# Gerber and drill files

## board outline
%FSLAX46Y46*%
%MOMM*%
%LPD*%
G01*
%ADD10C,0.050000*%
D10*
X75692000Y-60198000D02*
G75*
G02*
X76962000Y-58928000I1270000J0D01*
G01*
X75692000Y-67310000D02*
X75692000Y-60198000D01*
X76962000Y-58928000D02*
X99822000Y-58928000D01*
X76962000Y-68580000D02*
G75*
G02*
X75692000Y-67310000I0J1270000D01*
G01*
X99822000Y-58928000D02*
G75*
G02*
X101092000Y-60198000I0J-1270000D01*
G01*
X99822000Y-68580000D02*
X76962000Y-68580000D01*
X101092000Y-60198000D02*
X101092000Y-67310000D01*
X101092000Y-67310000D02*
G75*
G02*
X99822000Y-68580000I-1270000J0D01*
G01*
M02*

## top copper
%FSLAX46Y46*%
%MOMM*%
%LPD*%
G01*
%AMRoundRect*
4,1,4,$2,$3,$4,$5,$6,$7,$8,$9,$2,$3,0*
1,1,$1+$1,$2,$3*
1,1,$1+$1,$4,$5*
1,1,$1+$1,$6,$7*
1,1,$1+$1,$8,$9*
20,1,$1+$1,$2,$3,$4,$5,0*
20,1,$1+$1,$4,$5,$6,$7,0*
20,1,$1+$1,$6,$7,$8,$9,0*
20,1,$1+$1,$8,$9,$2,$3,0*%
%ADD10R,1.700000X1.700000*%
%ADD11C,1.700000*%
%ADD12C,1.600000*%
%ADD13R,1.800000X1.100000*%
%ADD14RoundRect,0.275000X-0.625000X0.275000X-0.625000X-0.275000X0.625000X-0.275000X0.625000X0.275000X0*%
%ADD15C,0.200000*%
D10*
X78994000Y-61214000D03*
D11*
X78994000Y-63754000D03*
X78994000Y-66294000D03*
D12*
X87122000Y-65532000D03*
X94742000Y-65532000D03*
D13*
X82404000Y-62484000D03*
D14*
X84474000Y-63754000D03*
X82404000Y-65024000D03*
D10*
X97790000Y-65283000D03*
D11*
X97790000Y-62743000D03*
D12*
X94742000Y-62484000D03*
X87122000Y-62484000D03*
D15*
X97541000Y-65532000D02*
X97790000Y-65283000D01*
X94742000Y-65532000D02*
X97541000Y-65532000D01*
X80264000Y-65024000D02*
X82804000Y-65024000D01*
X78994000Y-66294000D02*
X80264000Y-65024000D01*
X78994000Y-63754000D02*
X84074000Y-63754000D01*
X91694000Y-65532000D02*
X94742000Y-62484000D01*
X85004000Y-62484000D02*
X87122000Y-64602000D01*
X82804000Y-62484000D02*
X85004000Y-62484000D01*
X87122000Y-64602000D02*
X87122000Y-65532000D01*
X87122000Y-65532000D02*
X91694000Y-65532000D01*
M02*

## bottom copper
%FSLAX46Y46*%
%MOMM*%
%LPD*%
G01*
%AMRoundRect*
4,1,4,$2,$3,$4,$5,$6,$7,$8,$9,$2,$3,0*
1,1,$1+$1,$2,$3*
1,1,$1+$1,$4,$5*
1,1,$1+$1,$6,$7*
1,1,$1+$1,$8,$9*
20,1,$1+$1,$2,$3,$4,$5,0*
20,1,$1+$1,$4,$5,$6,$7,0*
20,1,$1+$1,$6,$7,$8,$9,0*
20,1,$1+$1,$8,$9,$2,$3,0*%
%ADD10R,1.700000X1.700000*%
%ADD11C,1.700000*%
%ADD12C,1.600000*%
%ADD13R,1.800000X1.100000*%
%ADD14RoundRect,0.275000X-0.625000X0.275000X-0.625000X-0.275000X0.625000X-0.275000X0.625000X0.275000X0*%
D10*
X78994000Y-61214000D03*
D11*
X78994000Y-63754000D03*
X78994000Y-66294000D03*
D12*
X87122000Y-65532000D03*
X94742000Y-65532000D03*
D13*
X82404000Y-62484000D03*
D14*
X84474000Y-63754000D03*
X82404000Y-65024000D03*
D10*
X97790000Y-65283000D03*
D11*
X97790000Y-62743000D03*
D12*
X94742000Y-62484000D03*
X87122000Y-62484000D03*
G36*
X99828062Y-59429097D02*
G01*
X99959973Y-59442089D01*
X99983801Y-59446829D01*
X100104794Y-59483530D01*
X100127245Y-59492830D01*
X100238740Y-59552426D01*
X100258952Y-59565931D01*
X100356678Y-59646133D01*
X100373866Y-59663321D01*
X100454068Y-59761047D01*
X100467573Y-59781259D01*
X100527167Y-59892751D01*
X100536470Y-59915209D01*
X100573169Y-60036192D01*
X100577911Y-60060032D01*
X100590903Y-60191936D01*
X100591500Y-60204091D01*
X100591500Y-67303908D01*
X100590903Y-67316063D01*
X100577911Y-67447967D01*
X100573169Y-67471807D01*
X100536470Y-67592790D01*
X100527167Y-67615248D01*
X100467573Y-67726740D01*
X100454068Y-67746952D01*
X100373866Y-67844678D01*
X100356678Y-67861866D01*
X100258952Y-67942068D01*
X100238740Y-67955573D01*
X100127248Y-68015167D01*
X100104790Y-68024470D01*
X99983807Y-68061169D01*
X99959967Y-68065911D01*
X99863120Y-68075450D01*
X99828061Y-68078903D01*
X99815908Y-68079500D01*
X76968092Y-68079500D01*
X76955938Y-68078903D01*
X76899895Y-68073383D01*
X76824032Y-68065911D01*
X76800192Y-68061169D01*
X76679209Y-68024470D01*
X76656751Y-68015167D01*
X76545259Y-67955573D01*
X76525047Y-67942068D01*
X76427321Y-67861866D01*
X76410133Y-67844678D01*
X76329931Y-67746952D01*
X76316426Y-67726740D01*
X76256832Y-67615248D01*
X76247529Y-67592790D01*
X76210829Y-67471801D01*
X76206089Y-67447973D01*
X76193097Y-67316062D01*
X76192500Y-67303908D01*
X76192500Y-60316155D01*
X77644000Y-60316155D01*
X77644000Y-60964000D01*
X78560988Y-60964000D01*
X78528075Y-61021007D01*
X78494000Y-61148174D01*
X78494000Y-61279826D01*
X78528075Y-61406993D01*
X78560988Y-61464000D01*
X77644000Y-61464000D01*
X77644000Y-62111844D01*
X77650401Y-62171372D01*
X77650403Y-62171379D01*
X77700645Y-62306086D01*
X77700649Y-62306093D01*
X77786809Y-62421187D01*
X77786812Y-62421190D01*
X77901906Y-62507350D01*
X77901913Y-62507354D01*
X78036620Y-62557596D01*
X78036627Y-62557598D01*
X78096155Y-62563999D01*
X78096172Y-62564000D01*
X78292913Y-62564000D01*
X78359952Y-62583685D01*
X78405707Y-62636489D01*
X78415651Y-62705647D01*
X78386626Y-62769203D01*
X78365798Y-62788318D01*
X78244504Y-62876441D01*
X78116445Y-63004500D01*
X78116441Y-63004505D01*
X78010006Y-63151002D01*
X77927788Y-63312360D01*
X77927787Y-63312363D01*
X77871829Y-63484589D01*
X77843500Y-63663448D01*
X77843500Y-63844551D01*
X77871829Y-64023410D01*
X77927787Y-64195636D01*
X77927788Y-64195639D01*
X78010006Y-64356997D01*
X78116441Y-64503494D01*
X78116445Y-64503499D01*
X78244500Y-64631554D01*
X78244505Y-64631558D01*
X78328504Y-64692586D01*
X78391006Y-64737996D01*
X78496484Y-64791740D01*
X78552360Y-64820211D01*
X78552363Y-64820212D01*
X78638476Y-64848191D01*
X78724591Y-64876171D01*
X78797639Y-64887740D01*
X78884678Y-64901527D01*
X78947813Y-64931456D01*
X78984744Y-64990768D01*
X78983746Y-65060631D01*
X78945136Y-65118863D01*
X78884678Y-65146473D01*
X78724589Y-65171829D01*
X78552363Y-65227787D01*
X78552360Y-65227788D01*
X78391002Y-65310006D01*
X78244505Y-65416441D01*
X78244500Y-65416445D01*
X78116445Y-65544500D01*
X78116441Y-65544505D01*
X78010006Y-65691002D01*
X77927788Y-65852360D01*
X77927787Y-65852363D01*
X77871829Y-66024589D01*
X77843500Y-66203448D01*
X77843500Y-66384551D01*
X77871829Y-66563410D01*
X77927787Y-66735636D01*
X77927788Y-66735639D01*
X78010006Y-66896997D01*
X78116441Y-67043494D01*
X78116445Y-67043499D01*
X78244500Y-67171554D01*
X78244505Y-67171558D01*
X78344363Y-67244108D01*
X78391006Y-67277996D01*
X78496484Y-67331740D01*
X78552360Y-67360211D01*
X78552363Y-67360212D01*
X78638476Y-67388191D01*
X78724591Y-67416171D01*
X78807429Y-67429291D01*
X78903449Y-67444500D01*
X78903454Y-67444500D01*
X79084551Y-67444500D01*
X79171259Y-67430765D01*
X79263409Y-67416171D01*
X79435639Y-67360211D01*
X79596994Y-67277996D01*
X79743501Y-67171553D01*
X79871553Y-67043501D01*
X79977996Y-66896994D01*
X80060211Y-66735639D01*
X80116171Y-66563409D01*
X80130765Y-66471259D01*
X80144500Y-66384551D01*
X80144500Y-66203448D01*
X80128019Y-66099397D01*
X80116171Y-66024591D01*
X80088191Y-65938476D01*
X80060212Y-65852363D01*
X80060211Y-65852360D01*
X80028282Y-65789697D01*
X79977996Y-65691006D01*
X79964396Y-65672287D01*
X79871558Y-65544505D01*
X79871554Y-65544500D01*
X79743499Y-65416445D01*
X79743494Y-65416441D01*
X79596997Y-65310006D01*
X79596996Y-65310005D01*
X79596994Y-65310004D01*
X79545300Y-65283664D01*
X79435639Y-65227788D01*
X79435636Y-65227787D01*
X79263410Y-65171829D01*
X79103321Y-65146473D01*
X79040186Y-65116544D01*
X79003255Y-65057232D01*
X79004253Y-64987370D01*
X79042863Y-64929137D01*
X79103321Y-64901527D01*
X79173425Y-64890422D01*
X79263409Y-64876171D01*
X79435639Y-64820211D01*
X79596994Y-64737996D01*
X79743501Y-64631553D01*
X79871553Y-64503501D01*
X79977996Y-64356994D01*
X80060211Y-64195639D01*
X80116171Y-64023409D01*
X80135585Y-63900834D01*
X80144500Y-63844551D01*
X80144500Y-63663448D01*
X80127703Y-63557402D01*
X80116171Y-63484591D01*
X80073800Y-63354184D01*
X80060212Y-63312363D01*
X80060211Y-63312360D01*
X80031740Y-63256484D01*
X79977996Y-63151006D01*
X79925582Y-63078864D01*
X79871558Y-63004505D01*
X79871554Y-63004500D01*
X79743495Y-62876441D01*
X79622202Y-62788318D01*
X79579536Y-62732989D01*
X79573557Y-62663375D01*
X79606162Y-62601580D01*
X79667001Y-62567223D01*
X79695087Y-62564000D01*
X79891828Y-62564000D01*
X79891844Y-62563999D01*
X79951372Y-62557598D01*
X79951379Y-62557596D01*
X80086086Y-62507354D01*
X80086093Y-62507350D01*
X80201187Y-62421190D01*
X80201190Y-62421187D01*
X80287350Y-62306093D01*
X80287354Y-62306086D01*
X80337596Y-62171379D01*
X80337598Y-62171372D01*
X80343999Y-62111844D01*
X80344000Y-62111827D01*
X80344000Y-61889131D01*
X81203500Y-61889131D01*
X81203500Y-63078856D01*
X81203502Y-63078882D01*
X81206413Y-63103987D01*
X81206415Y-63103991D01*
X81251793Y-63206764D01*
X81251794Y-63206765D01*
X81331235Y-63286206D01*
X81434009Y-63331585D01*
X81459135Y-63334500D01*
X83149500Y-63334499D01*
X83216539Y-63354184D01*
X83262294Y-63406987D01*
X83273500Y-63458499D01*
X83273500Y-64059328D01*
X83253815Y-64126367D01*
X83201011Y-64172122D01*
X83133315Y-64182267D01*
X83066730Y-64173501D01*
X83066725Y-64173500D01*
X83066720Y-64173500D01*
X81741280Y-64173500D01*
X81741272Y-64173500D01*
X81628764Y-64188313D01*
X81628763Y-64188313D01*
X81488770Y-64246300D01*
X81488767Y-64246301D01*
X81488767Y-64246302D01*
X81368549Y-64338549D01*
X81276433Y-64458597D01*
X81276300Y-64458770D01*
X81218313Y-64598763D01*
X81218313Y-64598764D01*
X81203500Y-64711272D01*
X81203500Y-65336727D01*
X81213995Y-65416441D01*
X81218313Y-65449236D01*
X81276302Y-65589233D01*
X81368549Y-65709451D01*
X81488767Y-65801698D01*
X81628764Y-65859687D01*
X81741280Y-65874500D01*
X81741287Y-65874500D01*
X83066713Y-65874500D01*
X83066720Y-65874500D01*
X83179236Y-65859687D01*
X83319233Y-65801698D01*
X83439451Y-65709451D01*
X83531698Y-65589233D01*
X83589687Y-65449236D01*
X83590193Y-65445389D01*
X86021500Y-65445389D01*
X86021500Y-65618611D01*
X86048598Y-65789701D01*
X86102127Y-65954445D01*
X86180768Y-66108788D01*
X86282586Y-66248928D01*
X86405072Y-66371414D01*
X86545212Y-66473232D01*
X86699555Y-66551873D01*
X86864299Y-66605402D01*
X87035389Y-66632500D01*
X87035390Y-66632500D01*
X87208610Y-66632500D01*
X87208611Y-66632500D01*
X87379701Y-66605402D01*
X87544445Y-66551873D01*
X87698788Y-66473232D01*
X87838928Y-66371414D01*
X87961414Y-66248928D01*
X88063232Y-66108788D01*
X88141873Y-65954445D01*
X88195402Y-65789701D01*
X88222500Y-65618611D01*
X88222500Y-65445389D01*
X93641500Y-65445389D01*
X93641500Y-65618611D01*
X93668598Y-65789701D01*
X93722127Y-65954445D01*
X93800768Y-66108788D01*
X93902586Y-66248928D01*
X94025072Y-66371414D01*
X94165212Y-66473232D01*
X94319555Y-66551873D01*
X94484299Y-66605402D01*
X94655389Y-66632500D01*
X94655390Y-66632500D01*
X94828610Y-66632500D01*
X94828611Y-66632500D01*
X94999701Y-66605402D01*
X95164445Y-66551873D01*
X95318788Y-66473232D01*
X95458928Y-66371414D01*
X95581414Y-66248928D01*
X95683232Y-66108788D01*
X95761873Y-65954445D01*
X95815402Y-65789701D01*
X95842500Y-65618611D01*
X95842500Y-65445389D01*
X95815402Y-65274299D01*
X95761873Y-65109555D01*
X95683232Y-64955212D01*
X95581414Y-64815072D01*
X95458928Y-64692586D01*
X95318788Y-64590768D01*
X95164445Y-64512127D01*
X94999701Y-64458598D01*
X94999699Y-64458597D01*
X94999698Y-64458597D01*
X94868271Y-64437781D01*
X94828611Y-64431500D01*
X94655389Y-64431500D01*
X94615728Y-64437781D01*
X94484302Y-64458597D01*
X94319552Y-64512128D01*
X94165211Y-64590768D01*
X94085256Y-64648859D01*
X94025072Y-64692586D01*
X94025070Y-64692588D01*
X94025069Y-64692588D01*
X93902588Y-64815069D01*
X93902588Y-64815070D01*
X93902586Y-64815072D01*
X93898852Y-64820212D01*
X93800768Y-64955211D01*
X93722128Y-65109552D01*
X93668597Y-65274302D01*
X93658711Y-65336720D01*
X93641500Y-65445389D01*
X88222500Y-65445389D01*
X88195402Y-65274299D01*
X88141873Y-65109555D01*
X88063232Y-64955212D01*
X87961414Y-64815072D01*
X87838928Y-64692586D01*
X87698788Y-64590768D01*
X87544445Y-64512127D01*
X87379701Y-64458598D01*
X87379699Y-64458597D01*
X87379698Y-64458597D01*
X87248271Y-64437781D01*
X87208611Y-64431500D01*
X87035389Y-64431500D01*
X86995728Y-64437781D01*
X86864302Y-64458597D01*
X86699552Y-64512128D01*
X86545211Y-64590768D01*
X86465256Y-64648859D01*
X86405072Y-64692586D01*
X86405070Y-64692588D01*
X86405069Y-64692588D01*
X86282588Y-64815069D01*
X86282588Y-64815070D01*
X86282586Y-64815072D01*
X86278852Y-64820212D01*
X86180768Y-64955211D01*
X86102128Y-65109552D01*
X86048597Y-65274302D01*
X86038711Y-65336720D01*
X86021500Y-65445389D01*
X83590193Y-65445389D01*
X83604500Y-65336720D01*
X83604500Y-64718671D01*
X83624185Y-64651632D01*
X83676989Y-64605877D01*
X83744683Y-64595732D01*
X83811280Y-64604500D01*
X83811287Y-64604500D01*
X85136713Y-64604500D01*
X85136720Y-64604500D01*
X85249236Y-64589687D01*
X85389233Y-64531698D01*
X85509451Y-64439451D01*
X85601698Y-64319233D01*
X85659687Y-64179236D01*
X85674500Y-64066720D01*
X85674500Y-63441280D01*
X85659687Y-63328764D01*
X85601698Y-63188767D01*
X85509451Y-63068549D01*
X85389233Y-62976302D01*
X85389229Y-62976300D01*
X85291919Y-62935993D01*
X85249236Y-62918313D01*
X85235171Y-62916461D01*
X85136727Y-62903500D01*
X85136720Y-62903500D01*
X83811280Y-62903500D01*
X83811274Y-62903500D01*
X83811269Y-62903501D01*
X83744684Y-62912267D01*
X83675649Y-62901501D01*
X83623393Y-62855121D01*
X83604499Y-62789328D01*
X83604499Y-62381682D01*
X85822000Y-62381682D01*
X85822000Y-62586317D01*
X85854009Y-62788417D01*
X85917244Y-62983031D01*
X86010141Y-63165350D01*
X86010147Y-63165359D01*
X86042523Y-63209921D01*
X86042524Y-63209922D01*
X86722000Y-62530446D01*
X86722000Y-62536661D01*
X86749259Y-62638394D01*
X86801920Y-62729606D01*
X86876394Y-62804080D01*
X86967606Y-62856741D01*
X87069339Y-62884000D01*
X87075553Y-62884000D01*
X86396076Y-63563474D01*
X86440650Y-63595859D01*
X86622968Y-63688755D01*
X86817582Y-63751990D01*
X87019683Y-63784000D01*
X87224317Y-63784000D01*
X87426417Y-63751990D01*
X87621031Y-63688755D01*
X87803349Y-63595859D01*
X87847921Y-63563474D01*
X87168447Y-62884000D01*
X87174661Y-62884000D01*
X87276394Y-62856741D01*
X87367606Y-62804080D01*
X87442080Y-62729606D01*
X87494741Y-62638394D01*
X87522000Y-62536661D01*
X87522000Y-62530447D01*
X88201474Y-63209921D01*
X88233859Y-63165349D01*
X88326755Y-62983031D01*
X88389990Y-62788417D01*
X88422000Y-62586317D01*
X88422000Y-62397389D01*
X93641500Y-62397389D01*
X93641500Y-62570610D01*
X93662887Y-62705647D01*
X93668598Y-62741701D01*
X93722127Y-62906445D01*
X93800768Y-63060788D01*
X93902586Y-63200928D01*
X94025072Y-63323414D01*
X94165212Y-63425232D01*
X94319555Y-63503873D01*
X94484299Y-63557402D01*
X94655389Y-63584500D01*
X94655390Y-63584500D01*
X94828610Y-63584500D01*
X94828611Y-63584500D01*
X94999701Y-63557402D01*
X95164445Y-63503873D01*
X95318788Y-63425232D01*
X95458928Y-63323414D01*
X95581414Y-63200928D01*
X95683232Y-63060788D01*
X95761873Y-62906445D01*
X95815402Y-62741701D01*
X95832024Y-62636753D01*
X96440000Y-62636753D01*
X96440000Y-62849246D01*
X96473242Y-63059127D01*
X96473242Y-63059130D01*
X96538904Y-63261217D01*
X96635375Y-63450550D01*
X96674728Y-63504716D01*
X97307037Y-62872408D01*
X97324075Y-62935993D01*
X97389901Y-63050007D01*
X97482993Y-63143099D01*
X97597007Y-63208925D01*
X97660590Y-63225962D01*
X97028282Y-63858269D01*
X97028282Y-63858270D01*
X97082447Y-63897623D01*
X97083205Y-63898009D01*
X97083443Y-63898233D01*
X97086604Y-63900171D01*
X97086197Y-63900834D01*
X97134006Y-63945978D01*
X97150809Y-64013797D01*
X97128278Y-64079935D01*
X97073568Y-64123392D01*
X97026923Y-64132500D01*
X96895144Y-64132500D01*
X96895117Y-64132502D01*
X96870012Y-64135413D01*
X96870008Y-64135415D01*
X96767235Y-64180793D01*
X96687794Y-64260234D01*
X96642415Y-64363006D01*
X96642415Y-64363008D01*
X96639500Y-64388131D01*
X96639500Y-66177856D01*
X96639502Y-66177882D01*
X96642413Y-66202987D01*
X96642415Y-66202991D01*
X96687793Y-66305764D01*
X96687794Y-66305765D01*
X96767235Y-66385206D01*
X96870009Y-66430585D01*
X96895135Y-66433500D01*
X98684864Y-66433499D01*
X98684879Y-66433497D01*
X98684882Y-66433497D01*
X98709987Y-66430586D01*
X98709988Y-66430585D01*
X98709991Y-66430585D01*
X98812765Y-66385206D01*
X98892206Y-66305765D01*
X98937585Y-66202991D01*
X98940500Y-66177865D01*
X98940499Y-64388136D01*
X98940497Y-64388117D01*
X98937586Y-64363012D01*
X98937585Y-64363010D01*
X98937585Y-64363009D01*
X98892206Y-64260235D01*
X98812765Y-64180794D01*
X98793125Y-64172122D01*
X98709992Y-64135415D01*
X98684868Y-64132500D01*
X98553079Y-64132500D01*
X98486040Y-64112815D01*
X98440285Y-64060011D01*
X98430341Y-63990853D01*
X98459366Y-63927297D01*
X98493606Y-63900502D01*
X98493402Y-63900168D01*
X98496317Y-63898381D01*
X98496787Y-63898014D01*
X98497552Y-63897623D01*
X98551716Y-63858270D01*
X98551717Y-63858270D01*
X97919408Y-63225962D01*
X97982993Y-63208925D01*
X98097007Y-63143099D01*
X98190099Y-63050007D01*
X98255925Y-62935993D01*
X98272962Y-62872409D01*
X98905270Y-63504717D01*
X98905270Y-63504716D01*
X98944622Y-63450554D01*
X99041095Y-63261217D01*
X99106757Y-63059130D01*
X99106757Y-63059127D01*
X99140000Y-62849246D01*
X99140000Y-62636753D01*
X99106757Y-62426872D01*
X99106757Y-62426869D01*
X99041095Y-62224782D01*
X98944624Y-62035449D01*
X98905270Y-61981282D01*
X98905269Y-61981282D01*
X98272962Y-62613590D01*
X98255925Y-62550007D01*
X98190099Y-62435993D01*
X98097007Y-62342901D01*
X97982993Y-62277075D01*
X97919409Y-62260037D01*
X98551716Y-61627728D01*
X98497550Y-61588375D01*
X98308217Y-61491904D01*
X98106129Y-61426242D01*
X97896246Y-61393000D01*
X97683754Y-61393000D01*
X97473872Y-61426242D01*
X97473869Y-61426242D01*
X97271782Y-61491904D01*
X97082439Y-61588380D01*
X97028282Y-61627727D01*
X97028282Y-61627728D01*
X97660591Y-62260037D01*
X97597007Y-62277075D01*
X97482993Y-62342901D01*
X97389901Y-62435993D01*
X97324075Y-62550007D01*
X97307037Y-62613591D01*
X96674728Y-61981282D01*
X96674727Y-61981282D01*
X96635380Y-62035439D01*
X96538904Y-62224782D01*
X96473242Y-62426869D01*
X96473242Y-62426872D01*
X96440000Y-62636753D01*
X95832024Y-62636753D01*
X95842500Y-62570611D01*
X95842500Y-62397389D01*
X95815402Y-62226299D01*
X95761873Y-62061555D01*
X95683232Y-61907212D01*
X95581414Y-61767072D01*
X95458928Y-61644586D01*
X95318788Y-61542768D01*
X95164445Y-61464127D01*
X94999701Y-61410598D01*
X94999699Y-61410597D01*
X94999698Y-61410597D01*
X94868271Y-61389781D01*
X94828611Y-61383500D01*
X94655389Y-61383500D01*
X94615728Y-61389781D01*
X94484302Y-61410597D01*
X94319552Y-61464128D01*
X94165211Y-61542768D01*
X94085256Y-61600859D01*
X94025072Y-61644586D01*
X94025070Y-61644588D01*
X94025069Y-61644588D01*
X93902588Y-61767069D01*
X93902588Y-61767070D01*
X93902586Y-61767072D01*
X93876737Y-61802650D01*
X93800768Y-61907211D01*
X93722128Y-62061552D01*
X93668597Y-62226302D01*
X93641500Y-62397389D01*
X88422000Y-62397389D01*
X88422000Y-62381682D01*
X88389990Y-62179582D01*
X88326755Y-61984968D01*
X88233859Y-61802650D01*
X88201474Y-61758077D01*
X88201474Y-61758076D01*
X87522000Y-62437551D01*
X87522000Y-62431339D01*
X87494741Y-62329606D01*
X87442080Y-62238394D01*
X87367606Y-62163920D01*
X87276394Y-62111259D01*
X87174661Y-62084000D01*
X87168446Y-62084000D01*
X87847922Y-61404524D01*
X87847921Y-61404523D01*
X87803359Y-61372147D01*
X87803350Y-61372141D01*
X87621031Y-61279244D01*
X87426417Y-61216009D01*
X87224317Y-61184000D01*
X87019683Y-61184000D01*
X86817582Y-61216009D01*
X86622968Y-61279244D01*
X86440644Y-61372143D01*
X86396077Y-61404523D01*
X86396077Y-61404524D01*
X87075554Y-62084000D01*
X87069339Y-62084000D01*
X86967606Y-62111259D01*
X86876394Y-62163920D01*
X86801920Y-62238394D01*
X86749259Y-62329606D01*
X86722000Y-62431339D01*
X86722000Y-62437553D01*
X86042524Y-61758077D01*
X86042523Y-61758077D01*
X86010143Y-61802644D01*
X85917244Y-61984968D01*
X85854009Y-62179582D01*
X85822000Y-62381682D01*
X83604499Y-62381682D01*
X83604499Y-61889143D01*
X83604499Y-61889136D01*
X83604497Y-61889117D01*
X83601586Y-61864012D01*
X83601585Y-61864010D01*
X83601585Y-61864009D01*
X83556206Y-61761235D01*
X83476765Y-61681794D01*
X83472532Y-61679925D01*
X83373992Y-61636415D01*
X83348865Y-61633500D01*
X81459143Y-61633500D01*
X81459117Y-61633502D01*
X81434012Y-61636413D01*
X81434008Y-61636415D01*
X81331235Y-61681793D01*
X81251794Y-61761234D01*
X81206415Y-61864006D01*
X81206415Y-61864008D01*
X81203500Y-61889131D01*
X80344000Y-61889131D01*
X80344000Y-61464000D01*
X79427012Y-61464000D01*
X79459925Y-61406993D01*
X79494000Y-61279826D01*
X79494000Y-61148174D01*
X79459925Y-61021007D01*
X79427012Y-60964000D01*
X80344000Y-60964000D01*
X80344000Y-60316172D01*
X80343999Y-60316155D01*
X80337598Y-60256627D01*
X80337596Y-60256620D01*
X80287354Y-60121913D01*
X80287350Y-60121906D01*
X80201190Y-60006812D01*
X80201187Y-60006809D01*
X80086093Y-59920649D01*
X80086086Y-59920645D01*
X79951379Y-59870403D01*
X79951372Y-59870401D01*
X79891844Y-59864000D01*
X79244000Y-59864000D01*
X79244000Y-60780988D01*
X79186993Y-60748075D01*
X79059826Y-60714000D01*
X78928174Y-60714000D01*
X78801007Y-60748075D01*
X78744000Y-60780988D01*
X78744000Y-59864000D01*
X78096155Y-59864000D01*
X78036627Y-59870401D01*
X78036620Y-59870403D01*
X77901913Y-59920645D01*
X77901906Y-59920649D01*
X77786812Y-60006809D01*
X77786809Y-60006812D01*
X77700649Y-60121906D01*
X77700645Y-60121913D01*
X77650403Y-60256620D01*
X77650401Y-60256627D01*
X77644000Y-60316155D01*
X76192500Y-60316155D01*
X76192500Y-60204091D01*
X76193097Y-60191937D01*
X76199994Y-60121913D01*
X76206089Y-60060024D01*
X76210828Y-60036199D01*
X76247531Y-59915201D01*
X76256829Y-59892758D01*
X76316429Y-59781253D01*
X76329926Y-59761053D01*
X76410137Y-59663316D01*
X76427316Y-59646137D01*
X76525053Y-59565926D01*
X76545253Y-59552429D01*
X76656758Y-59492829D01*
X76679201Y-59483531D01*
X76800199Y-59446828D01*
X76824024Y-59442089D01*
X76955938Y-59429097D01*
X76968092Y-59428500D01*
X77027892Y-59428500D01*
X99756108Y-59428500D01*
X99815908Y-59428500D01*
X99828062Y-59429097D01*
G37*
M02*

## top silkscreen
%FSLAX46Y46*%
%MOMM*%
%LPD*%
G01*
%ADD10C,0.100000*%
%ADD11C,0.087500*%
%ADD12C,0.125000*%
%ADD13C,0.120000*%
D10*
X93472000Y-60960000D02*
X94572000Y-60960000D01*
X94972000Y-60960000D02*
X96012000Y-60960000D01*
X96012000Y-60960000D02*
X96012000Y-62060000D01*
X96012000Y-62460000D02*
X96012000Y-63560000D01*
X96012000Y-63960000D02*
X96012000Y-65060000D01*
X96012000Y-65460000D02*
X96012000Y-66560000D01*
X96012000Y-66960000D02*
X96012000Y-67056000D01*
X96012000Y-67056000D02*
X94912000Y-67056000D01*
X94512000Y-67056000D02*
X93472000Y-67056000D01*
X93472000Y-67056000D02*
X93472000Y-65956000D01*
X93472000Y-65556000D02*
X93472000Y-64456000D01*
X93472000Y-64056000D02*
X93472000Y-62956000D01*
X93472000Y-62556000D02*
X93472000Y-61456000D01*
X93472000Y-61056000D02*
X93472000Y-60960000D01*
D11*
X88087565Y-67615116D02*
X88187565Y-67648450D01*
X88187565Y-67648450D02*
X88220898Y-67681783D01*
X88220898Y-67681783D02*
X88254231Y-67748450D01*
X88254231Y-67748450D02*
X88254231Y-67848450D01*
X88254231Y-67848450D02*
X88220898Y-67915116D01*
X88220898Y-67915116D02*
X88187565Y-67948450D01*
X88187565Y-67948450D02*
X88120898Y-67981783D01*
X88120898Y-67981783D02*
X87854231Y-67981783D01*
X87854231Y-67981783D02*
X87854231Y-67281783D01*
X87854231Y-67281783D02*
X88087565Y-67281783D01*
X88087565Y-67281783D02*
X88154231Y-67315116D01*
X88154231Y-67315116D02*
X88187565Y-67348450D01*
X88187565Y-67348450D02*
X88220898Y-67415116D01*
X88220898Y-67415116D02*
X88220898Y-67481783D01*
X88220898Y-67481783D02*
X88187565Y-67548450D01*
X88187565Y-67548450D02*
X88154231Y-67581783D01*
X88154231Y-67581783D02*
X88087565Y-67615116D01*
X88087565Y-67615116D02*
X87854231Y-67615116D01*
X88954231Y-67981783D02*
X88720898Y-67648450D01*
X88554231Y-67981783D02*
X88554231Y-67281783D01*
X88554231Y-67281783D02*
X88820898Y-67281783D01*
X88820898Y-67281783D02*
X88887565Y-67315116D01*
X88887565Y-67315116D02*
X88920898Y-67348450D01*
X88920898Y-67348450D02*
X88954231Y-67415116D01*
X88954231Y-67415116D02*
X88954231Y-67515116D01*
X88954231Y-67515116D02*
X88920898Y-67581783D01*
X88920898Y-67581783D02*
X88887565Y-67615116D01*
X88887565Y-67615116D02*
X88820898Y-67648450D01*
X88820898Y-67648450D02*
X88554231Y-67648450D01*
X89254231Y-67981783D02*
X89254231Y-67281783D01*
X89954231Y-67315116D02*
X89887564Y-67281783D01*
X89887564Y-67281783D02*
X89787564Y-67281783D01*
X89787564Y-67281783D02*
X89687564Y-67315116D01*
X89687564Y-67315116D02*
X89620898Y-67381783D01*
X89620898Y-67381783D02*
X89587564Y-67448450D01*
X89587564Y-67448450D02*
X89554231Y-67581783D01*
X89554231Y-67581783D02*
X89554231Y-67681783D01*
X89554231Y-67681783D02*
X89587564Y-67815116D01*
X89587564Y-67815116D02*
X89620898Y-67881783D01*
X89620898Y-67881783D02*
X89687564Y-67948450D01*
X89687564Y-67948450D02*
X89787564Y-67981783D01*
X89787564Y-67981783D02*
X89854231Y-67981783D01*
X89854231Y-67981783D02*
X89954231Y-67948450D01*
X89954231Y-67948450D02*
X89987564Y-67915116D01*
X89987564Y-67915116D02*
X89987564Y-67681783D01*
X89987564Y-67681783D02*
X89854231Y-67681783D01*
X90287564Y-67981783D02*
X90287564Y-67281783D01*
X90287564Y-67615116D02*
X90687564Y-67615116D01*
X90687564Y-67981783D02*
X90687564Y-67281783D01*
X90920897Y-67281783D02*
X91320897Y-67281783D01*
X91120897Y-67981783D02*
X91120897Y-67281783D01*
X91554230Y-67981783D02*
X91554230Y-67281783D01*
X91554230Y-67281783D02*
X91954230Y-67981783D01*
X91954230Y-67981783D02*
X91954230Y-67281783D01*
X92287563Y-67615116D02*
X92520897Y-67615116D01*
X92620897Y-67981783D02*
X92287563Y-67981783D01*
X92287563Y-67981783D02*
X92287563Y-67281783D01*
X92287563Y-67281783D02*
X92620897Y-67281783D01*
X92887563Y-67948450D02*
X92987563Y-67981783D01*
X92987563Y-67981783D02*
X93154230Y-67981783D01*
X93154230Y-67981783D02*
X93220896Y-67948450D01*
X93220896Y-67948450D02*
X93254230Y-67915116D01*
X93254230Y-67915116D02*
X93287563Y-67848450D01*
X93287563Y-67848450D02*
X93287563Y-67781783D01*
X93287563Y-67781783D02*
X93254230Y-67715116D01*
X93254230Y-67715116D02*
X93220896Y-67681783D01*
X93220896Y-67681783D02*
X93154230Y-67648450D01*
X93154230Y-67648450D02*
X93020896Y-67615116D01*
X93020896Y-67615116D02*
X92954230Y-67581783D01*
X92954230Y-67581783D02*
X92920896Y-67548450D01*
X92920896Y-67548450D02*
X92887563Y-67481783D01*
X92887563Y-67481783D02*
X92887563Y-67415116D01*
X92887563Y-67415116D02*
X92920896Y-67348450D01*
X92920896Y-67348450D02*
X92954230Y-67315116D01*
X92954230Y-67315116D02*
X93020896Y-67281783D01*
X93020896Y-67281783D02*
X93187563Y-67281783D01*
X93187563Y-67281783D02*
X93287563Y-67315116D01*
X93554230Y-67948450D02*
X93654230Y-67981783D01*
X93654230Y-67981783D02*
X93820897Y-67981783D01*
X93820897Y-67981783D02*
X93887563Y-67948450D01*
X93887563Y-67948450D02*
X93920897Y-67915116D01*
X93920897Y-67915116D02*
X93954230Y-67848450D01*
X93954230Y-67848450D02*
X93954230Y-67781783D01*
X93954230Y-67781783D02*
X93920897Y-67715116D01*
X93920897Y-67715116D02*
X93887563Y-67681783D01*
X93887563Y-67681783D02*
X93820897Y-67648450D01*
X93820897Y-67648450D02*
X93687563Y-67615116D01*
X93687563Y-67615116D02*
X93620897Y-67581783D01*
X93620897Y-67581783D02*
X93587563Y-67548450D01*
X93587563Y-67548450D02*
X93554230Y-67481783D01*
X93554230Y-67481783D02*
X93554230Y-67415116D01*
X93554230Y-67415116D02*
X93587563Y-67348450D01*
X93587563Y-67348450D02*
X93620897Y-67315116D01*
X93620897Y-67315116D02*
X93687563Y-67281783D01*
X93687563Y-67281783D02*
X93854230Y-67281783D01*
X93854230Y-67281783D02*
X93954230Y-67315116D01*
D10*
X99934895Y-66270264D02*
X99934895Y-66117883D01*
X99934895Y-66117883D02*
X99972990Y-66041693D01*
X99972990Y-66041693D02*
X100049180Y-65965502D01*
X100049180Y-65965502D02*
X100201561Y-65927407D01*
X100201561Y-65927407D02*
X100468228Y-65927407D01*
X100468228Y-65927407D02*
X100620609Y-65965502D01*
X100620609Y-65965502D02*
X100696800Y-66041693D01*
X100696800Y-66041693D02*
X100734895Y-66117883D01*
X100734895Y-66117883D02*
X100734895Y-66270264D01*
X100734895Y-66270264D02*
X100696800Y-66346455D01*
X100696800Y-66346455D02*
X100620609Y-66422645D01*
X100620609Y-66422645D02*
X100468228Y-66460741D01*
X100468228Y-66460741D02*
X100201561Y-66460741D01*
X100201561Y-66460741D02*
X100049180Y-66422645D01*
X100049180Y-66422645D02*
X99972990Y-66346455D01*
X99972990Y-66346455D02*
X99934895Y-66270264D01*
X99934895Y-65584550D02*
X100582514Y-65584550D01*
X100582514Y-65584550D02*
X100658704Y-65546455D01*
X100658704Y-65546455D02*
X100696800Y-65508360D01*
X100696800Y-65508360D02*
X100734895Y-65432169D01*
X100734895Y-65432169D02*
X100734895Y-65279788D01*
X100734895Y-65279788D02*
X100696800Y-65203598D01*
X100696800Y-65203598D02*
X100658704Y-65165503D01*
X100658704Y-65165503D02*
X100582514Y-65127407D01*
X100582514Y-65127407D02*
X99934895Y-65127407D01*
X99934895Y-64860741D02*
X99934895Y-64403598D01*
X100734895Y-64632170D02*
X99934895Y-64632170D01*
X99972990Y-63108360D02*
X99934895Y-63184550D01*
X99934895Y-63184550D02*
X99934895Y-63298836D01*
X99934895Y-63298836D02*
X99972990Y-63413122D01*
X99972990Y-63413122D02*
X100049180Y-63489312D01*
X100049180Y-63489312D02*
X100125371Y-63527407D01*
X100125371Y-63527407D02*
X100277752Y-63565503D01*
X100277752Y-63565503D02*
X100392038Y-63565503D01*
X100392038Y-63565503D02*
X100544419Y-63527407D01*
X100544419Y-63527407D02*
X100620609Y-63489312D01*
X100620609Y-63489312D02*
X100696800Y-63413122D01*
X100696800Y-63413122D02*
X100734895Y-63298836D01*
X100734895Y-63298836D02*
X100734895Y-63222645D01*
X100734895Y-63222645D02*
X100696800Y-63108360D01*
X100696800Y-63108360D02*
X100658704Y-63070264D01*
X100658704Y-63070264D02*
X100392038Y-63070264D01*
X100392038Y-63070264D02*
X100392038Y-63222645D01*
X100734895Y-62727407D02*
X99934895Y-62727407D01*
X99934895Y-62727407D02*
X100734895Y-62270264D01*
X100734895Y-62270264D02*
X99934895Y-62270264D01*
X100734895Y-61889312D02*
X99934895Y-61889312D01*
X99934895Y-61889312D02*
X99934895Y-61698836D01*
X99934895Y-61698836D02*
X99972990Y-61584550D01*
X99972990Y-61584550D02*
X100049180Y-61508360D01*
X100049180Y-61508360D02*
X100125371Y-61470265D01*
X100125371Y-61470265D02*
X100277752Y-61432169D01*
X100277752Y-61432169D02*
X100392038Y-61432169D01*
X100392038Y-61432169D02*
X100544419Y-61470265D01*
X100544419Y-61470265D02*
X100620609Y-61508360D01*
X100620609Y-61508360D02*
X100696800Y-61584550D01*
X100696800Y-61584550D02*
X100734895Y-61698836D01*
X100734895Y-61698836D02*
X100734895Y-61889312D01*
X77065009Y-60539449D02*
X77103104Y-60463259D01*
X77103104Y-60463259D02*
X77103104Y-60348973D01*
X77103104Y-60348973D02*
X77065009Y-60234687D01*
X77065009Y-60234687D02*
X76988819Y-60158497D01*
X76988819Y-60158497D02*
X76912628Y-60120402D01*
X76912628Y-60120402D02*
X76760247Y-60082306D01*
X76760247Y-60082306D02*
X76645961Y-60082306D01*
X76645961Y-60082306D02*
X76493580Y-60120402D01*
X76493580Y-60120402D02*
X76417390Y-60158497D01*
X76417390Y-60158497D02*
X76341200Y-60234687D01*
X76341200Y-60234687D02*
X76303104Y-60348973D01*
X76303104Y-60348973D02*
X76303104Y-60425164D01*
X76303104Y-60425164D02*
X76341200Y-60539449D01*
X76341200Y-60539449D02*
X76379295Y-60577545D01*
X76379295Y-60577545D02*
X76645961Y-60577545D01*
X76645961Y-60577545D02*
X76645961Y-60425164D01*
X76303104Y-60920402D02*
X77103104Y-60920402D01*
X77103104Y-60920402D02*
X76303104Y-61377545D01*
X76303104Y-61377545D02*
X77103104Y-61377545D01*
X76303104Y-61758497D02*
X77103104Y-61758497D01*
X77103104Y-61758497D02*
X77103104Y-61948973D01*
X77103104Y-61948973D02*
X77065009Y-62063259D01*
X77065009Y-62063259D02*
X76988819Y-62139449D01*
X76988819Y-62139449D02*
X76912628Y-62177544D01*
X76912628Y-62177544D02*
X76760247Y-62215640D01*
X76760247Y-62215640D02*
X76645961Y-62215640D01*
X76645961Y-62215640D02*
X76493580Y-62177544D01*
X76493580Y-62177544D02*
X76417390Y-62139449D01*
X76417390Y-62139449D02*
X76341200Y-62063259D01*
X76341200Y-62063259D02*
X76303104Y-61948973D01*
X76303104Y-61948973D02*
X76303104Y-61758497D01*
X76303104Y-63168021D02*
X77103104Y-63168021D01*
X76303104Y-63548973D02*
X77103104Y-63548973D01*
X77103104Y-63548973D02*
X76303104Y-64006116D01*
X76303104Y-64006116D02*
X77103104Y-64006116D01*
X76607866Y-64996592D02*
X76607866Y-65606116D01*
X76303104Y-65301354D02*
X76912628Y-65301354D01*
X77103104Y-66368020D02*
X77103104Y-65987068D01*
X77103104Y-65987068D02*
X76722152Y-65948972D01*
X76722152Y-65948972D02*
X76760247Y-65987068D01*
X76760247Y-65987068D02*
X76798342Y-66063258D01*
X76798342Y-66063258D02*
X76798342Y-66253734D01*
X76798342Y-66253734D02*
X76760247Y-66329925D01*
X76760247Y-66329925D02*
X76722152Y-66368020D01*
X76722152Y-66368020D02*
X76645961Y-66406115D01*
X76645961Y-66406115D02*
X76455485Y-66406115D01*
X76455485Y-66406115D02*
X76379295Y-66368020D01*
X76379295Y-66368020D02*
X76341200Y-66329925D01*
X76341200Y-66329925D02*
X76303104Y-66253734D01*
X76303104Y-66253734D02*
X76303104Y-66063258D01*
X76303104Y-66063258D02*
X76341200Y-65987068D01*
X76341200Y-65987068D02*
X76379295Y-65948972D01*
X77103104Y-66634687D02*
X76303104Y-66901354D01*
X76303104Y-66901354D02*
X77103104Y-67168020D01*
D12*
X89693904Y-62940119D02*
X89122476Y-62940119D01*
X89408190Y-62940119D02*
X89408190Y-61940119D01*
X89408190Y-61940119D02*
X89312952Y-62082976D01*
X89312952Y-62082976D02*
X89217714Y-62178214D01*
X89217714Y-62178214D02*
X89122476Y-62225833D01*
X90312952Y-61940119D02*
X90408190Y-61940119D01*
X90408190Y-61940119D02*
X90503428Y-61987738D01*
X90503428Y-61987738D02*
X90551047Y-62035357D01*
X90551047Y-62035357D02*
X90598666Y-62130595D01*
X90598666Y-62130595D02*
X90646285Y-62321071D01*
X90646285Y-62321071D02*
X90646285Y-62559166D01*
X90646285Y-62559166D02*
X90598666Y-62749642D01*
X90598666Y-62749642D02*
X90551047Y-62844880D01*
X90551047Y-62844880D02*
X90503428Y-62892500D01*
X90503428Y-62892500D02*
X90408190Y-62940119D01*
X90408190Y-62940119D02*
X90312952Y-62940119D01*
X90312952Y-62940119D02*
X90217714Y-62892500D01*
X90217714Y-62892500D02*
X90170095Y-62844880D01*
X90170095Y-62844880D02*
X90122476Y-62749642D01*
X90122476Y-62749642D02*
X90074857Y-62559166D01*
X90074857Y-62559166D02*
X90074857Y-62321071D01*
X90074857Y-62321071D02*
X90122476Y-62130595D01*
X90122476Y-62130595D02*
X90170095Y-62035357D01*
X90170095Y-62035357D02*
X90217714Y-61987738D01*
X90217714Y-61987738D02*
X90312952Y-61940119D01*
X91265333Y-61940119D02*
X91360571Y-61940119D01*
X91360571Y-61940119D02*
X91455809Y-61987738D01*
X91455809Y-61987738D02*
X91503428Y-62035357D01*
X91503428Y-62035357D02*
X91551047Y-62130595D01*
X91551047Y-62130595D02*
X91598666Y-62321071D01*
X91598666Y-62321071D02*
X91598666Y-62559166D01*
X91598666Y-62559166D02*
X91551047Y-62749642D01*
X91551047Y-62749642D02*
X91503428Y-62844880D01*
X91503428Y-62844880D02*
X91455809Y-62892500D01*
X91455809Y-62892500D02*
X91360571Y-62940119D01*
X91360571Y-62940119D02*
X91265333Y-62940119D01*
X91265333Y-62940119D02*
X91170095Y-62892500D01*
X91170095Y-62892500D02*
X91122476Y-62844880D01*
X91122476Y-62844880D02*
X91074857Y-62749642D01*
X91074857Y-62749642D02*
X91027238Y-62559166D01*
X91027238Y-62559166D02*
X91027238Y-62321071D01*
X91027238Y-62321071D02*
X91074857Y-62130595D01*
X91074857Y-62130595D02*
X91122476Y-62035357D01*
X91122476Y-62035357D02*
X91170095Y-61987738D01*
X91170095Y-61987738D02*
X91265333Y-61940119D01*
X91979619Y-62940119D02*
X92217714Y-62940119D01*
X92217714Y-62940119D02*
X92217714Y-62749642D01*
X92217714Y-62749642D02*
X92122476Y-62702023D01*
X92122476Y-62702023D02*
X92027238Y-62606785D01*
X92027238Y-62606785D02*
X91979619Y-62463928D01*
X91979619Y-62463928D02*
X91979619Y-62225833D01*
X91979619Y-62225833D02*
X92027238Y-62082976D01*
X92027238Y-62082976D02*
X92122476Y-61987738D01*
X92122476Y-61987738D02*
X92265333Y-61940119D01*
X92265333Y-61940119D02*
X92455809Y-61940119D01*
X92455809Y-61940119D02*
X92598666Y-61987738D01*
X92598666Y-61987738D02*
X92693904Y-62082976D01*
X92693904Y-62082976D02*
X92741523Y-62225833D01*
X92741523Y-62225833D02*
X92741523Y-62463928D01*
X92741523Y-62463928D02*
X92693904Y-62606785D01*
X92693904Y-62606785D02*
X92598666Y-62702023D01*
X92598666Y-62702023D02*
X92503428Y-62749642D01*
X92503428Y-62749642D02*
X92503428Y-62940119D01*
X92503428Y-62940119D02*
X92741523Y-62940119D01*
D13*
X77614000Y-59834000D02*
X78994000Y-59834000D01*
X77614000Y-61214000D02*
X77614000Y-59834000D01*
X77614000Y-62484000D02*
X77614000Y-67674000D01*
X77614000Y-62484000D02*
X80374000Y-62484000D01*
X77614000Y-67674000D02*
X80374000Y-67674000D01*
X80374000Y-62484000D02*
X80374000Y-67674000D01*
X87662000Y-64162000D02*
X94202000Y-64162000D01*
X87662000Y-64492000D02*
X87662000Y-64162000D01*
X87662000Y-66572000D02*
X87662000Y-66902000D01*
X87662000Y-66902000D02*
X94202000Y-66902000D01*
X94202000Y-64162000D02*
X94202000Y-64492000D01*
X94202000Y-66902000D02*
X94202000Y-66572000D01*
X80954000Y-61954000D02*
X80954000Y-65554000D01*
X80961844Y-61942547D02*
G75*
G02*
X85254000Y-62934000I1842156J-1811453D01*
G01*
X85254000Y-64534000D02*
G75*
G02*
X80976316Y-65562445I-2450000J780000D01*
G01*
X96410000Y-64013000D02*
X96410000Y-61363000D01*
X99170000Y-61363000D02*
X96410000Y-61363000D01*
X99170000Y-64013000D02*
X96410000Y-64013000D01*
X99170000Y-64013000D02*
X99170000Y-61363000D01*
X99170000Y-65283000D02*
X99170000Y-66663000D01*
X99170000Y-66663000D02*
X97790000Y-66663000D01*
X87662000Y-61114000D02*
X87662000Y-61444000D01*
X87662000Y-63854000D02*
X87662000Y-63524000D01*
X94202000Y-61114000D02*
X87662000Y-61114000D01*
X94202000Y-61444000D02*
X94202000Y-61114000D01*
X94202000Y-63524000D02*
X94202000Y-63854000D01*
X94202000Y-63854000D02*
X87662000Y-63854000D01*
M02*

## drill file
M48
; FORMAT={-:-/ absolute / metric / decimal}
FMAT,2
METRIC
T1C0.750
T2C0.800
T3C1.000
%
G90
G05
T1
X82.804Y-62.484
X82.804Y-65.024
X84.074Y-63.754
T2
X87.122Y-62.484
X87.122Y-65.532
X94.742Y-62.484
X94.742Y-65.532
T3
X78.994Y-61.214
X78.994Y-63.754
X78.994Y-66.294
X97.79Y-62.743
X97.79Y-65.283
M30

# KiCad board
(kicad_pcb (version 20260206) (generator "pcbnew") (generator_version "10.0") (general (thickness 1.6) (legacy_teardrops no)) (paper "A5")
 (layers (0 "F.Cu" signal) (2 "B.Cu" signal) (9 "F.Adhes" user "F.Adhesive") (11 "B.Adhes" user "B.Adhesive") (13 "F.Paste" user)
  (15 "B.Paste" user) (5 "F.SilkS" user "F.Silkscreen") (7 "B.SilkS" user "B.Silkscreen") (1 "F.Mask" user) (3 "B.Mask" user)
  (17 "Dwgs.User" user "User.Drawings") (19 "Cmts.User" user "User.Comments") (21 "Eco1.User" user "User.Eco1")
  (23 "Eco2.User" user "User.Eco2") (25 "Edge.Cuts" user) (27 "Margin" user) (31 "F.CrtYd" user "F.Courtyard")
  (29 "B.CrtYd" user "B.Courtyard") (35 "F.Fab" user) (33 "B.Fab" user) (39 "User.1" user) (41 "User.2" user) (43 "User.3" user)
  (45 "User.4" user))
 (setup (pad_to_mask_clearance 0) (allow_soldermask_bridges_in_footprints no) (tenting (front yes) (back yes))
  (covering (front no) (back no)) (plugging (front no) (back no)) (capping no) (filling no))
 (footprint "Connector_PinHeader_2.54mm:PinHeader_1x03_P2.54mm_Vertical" (layer "F.Cu") (at 78.994 61.214)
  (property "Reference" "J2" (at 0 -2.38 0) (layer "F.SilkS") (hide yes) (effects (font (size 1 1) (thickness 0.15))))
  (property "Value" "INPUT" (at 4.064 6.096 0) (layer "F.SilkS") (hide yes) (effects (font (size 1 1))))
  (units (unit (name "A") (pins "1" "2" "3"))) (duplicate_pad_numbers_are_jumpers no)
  (fp_line (start -1.38 -1.38) (end 0 -1.38) (stroke (width 0.12) (type solid)) (layer "F.SilkS"))
  (fp_line (start -1.38 0) (end -1.38 -1.38) (stroke (width 0.12) (type solid)) (layer "F.SilkS"))
  (fp_line (start -1.38 1.27) (end -1.38 6.46) (stroke (width 0.12) (type solid)) (layer "F.SilkS"))
  (fp_line (start -1.38 1.27) (end 1.38 1.27) (stroke (width 0.12) (type solid)) (layer "F.SilkS"))
  (fp_line (start -1.38 6.46) (end 1.38 6.46) (stroke (width 0.12) (type solid)) (layer "F.SilkS"))
  (fp_line (start 1.38 1.27) (end 1.38 6.46) (stroke (width 0.12) (type solid)) (layer "F.SilkS"))
  (pad "1" thru_hole rect (at 0 0) (size 1.7 1.7) (drill 1) (layers "*.Cu" "*.Mask") (remove_unused_layers no) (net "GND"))
  (pad "2" thru_hole circle (at 0 2.54) (size 1.7 1.7) (drill 1) (layers "*.Cu" "*.Mask") (remove_unused_layers no) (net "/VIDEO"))
  (pad "3" thru_hole circle (at 0 5.08) (size 1.7 1.7) (drill 1) (layers "*.Cu" "*.Mask") (remove_unused_layers no) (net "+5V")))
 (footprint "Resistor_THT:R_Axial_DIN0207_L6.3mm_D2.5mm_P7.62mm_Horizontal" (layer "F.Cu") (at 87.122 65.532)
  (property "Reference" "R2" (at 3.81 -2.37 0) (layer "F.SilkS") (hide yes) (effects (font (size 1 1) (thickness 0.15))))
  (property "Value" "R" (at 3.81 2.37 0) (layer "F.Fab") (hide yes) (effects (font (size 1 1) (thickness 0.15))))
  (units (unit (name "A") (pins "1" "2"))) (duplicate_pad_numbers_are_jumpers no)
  (fp_line (start 0.54 -1.37) (end 7.08 -1.37) (stroke (width 0.12) (type solid)) (layer "F.SilkS"))
  (fp_line (start 0.54 -1.04) (end 0.54 -1.37) (stroke (width 0.12) (type solid)) (layer "F.SilkS"))
  (fp_line (start 0.54 1.04) (end 0.54 1.37) (stroke (width 0.12) (type solid)) (layer "F.SilkS"))
  (fp_line (start 0.54 1.37) (end 7.08 1.37) (stroke (width 0.12) (type solid)) (layer "F.SilkS"))
  (fp_line (start 7.08 -1.37) (end 7.08 -1.04) (stroke (width 0.12) (type solid)) (layer "F.SilkS"))
  (fp_line (start 7.08 1.37) (end 7.08 1.04) (stroke (width 0.12) (type solid)) (layer "F.SilkS"))
  (pad "1" thru_hole circle (at 0 0) (size 1.6 1.6) (drill 0.8) (layers "*.Cu" "*.Mask") (remove_unused_layers no) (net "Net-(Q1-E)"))
  (pad "2" thru_hole circle (at 7.62 0) (size 1.6 1.6) (drill 0.8) (layers "*.Cu" "*.Mask") (remove_unused_layers no) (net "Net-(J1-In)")))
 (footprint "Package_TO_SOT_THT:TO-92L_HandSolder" (layer "F.Cu") (at 82.804 62.484 -90)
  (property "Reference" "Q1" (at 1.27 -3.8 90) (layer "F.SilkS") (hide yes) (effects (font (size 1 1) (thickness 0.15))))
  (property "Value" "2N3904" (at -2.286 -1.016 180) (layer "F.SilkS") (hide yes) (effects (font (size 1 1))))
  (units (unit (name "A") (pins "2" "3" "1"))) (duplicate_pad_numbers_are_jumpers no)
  (fp_line (start -0.53 1.85) (end 3.07 1.85) (stroke (width 0.12) (type solid)) (layer "F.SilkS"))
  (fp_arc (start -0.541453 1.842156) (mid -1.247298 -0.581475) (end 0.45 -2.45) (stroke (width 0.12) (type solid)) (layer "F.SilkS"))
  (fp_arc (start 2.05 -2.45) (mid 3.769931 -0.601036) (end 3.078445 1.827684) (stroke (width 0.12) (type solid)) (layer "F.SilkS"))
  (pad "1" thru_hole rect (at 0 0 270) (size 1.1 1.8) (drill 0.75 (offset 0 0.4)) (layers "*.Cu" "*.Mask") (remove_unused_layers no)
   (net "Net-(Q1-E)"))
  (pad "2" thru_hole roundrect (at 1.27 -1.27 270) (size 1.1 1.8) (drill 0.75 (offset 0 -0.4)) (layers "*.Cu" "*.Mask")
   (remove_unused_layers no) (roundrect_rratio 0.25) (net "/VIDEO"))
  (pad "3" thru_hole roundrect (at 2.54 0 270) (size 1.1 1.8) (drill 0.75 (offset 0 0.4)) (layers "*.Cu" "*.Mask") (remove_unused_layers no)
   (roundrect_rratio 0.25) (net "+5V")))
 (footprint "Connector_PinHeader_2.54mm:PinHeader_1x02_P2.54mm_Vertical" (layer "F.Cu") (at 97.79 65.283 180)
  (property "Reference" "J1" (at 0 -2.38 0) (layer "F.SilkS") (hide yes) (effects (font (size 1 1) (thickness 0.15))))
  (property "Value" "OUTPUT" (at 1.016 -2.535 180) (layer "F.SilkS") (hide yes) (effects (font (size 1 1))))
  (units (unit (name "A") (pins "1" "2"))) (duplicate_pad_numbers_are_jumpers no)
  (fp_line (start 1.38 1.27) (end 1.38 3.92) (stroke (width 0.12) (type solid)) (layer "F.SilkS"))
  (fp_line (start -1.38 3.92) (end 1.38 3.92) (stroke (width 0.12) (type solid)) (layer "F.SilkS"))
  (fp_line (start -1.38 1.27) (end 1.38 1.27) (stroke (width 0.12) (type solid)) (layer "F.SilkS"))
  (fp_line (start -1.38 1.27) (end -1.38 3.92) (stroke (width 0.12) (type solid)) (layer "F.SilkS"))
  (fp_line (start -1.38 0) (end -1.38 -1.38) (stroke (width 0.12) (type solid)) (layer "F.SilkS"))
  (fp_line (start -1.38 -1.38) (end 0 -1.38) (stroke (width 0.12) (type solid)) (layer "F.SilkS"))
  (pad "1" thru_hole rect (at 0 0 180) (size 1.7 1.7) (drill 1) (layers "*.Cu" "*.Mask") (remove_unused_layers no) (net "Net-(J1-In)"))
  (pad "2" thru_hole circle (at 0 2.54 180) (size 1.7 1.7) (drill 1) (layers "*.Cu" "*.Mask") (remove_unused_layers no) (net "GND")))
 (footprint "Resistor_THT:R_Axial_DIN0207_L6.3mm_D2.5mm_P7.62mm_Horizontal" (layer "F.Cu") (at 94.742 62.484 180)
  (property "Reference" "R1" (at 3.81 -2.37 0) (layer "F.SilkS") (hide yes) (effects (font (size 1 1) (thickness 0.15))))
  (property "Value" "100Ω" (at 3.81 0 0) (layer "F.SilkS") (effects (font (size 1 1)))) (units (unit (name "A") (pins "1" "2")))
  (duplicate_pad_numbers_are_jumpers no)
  (fp_line (start 7.08 1.37) (end 7.08 1.04) (stroke (width 0.12) (type solid)) (layer "F.SilkS"))
  (fp_line (start 7.08 -1.37) (end 7.08 -1.04) (stroke (width 0.12) (type solid)) (layer "F.SilkS"))
  (fp_line (start 0.54 1.37) (end 7.08 1.37) (stroke (width 0.12) (type solid)) (layer "F.SilkS"))
  (fp_line (start 0.54 1.04) (end 0.54 1.37) (stroke (width 0.12) (type solid)) (layer "F.SilkS"))
  (fp_line (start 0.54 -1.04) (end 0.54 -1.37) (stroke (width 0.12) (type solid)) (layer "F.SilkS"))
  (fp_line (start 0.54 -1.37) (end 7.08 -1.37) (stroke (width 0.12) (type solid)) (layer "F.SilkS"))
  (pad "1" thru_hole circle (at 0 0 180) (size 1.6 1.6) (drill 0.8) (layers "*.Cu" "*.Mask") (remove_unused_layers no) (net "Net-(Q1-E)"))
  (pad "2" thru_hole circle (at 7.62 0 180) (size 1.6 1.6) (drill 0.8) (layers "*.Cu" "*.Mask") (remove_unused_layers no) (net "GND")))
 (gr_rect (start 93.472 60.96) (end 96.012 67.056) (stroke (width 0.1) (type dash)) (fill no) (layer "F.SilkS"))
 (gr_arc (start 75.692 60.198) (mid 76.063974 59.299974) (end 76.962 58.928) (stroke (width 0.05) (type default)) (layer "Edge.Cuts"))
 (gr_line (start 75.692 67.31) (end 75.692 60.198) (stroke (width 0.05) (type default)) (layer "Edge.Cuts"))
 (gr_line (start 76.962 58.928) (end 99.822 58.928) (stroke (width 0.05) (type default)) (layer "Edge.Cuts"))
 (gr_arc (start 76.962 68.58) (mid 76.063974 68.208026) (end 75.692 67.31) (stroke (width 0.05) (type default)) (layer "Edge.Cuts"))
 (gr_arc (start 99.822 58.928) (mid 100.720026 59.299974) (end 101.092 60.198) (stroke (width 0.05) (type default)) (layer "Edge.Cuts"))
 (gr_line (start 99.822 68.58) (end 76.962 68.58) (stroke (width 0.05) (type default)) (layer "Edge.Cuts"))
 (gr_line (start 101.092 60.198) (end 101.092 67.31) (stroke (width 0.05) (type default)) (layer "Edge.Cuts"))
 (gr_arc (start 101.092 67.31) (mid 100.720026 68.208026) (end 99.822 68.58) (stroke (width 0.05) (type default)) (layer "Edge.Cuts"))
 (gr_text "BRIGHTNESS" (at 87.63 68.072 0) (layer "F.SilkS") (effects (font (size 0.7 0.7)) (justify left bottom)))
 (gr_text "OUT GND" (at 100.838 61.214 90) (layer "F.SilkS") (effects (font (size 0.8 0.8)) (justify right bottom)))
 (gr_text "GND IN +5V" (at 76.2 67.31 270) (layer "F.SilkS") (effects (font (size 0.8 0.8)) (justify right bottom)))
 (segment (start 97.541 65.532) (end 97.79 65.283) (width 0.2) (layer "F.Cu") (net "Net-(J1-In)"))
 (segment (start 94.742 65.532) (end 97.541 65.532) (width 0.2) (layer "F.Cu") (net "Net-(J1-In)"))
 (segment (start 80.264 65.024) (end 82.804 65.024) (width 0.2) (layer "F.Cu") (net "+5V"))
 (segment (start 78.994 66.294) (end 80.264 65.024) (width 0.2) (layer "F.Cu") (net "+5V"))
 (segment (start 78.994 63.754) (end 84.074 63.754) (width 0.2) (layer "F.Cu") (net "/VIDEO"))
 (segment (start 91.694 65.532) (end 94.742 62.484) (width 0.2) (layer "F.Cu") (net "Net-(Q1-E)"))
 (segment (start 85.004 62.484) (end 87.122 64.602) (width 0.2) (layer "F.Cu") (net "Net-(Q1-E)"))
 (segment (start 82.804 62.484) (end 85.004 62.484) (width 0.2) (layer "F.Cu") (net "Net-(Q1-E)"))
 (segment (start 87.122 64.602) (end 87.122 65.532) (width 0.2) (layer "F.Cu") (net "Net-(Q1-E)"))
 (segment (start 87.122 65.532) (end 91.694 65.532) (width 0.2) (layer "F.Cu") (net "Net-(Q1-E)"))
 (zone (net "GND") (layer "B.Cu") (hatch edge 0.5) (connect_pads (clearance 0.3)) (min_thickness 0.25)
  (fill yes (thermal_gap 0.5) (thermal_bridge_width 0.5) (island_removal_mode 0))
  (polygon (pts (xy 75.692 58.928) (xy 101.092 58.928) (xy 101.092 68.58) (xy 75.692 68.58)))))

